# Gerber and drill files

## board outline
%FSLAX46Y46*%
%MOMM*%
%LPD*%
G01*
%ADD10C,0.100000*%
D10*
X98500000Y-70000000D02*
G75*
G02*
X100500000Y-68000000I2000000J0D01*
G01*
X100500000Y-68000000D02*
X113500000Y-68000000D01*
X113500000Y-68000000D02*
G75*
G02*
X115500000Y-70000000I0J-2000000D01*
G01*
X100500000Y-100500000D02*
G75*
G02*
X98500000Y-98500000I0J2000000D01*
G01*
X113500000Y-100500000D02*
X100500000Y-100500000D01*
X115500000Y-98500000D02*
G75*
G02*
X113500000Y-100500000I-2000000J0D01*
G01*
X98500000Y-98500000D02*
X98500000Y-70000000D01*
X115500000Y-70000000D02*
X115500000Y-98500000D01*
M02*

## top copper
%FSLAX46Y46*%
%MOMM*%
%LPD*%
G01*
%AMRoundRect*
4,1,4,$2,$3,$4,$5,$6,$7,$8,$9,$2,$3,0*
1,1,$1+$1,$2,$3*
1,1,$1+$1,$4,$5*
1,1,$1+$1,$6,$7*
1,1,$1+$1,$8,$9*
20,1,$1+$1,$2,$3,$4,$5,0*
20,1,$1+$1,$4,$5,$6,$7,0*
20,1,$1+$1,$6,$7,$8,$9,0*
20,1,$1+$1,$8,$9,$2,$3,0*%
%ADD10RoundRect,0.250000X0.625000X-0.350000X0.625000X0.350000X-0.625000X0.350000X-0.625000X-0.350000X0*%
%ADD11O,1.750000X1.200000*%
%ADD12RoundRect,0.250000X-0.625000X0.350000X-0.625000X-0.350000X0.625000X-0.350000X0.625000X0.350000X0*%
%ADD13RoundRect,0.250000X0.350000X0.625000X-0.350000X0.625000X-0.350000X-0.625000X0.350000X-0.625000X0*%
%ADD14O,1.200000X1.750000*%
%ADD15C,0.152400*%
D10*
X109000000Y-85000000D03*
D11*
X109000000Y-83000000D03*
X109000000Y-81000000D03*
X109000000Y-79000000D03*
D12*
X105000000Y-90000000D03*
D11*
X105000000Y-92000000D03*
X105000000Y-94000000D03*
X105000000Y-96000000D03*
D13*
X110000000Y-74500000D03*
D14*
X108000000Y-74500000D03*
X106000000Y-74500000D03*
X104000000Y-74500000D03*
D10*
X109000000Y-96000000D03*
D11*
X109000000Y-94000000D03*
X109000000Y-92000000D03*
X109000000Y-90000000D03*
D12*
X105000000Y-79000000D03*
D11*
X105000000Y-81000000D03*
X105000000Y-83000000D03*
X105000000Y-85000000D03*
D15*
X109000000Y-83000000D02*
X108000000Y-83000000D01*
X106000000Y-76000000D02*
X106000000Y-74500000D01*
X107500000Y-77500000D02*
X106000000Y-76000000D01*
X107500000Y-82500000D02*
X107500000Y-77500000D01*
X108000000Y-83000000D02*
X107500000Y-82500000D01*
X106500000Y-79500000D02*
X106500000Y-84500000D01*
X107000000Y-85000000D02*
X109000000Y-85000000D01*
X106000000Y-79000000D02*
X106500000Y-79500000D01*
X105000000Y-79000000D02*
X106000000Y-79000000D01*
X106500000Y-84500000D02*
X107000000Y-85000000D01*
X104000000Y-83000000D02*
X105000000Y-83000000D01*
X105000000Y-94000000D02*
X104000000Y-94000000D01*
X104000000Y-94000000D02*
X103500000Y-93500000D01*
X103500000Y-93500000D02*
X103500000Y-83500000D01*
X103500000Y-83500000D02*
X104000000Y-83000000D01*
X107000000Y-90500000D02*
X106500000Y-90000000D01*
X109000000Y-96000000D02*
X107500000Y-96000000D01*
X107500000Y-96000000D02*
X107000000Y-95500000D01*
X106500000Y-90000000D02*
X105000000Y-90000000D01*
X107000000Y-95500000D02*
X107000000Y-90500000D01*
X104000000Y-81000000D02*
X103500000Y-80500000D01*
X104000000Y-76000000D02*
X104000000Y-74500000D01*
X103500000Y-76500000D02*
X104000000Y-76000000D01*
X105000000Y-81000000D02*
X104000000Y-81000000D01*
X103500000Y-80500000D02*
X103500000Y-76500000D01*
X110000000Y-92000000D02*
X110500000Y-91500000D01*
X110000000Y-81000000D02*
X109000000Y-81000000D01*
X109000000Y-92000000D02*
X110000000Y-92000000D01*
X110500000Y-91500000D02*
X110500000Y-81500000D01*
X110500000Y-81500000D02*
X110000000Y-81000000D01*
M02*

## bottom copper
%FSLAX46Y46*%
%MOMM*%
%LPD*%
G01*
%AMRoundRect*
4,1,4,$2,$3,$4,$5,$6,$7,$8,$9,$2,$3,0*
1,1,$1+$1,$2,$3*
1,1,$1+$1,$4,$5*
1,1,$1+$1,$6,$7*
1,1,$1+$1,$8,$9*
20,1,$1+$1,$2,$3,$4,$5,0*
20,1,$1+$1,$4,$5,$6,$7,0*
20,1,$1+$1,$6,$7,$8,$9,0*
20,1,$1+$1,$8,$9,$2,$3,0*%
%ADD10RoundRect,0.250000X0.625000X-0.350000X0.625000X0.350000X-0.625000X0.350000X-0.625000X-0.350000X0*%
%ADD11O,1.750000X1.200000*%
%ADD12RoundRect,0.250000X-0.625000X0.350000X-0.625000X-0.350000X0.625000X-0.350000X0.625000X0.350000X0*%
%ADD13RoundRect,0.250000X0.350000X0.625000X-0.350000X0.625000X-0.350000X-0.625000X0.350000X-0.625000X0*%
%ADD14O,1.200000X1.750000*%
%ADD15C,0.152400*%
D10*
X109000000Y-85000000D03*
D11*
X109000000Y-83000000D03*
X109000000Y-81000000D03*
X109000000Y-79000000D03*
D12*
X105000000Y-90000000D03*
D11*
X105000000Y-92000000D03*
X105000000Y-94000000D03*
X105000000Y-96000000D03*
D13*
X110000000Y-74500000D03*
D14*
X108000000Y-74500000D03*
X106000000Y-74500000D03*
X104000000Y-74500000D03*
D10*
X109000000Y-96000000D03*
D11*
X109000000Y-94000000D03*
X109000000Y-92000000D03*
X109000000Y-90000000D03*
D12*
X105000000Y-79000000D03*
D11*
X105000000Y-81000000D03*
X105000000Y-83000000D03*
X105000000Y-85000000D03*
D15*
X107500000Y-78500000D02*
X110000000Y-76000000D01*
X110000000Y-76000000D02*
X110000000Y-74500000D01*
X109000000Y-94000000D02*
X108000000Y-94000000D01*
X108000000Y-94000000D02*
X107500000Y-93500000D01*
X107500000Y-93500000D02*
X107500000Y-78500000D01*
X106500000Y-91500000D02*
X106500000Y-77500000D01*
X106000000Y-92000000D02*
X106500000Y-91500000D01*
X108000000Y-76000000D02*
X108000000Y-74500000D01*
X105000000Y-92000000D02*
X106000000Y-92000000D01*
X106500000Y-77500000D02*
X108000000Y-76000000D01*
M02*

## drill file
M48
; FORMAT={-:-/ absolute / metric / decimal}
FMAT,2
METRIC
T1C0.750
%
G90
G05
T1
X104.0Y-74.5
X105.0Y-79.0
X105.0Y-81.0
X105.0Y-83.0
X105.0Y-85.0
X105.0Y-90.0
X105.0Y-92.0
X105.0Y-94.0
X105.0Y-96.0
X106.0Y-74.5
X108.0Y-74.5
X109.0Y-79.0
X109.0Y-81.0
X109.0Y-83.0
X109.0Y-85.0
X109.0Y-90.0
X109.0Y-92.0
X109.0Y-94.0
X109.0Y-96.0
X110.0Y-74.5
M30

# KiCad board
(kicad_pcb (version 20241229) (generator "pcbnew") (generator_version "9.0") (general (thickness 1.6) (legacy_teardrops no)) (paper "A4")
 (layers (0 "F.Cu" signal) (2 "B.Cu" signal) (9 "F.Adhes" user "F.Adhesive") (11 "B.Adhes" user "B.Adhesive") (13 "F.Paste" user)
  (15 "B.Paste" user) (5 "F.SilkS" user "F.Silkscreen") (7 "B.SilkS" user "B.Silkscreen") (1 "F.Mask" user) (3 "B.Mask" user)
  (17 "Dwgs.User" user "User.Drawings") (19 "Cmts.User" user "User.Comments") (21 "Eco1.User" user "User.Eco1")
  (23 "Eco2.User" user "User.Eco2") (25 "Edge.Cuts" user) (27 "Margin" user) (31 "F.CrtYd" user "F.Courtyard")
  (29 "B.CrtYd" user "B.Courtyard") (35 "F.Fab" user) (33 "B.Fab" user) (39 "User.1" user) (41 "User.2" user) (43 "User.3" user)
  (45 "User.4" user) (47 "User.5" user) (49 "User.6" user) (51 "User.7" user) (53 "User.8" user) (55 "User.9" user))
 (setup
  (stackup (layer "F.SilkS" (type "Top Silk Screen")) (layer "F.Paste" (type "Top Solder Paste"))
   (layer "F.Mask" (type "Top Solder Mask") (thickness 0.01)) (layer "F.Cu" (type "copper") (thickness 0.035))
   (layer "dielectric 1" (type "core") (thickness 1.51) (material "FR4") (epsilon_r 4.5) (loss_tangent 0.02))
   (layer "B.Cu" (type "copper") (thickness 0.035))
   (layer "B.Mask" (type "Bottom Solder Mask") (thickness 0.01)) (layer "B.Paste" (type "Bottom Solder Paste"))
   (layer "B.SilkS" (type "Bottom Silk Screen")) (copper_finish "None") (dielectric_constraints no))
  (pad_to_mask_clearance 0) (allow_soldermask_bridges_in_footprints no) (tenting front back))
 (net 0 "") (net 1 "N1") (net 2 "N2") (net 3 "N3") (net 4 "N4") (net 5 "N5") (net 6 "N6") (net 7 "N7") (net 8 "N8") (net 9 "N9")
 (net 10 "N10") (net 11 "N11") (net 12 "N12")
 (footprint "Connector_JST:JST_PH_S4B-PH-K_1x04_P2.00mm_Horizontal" (layer "F.Cu") (at 109 85 90)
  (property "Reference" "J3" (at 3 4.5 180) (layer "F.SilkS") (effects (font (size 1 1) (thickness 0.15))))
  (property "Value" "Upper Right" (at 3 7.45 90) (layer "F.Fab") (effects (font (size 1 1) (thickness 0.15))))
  (pad "1" thru_hole roundrect (at 0 0 90) (size 1.2 1.75) (drill 0.75) (layers "*.Cu" "*.Mask") (remove_unused_layers no)
   (roundrect_rratio 0.208333) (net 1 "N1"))
  (pad "2" thru_hole oval (at 2 0 90) (size 1.2 1.75) (drill 0.75) (layers "*.Cu" "*.Mask") (remove_unused_layers no) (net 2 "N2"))
  (pad "3" thru_hole oval (at 4 0 90) (size 1.2 1.75) (drill 0.75) (layers "*.Cu" "*.Mask") (remove_unused_layers no) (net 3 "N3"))
  (pad "4" thru_hole oval (at 6 0 90) (size 1.2 1.75) (drill 0.75) (layers "*.Cu" "*.Mask") (remove_unused_layers no) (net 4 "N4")))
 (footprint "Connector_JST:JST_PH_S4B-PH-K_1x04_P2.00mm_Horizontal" (layer "F.Cu") (at 105 90 -90)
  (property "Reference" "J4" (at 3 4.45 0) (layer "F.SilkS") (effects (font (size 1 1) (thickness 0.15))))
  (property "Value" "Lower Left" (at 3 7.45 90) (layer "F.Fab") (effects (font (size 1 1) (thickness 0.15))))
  (pad "1" thru_hole roundrect (at 0 0 270) (size 1.2 1.75) (drill 0.75) (layers "*.Cu" "*.Mask") (remove_unused_layers no)
   (roundrect_rratio 0.208333) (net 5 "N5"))
  (pad "2" thru_hole oval (at 2 0 270) (size 1.2 1.75) (drill 0.75) (layers "*.Cu" "*.Mask") (remove_unused_layers no) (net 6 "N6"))
  (pad "3" thru_hole oval (at 4 0 270) (size 1.2 1.75) (drill 0.75) (layers "*.Cu" "*.Mask") (remove_unused_layers no) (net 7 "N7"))
  (pad "4" thru_hole oval (at 6 0 270) (size 1.2 1.75) (drill 0.75) (layers "*.Cu" "*.Mask") (remove_unused_layers no) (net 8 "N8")))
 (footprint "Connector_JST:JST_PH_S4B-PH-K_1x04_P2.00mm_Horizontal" (layer "F.Cu") (at 110 74.5 180)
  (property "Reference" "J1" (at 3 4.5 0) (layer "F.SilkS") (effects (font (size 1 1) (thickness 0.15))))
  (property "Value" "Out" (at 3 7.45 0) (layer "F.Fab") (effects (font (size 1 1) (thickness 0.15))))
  (pad "1" thru_hole roundrect (at 0 0 180) (size 1.2 1.75) (drill 0.75) (layers "*.Cu" "*.Mask") (remove_unused_layers no)
   (roundrect_rratio 0.208333) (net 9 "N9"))
  (pad "2" thru_hole oval (at 2 0 180) (size 1.2 1.75) (drill 0.75) (layers "*.Cu" "*.Mask") (remove_unused_layers no) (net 6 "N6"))
  (pad "3" thru_hole oval (at 4 0 180) (size 1.2 1.75) (drill 0.75) (layers "*.Cu" "*.Mask") (remove_unused_layers no) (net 2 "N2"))
  (pad "4" thru_hole oval (at 6 0 180) (size 1.2 1.75) (drill 0.75) (layers "*.Cu" "*.Mask") (remove_unused_layers no) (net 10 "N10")))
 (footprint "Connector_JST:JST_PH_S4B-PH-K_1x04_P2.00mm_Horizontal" (layer "F.Cu") (at 109 96 90)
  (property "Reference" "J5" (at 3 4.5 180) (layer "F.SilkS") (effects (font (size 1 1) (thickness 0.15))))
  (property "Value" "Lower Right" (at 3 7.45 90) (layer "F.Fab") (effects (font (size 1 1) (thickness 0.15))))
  (pad "1" thru_hole roundrect (at 0 0 90) (size 1.2 1.75) (drill 0.75) (layers "*.Cu" "*.Mask") (remove_unused_layers no)
   (roundrect_rratio 0.208333) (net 5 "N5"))
  (pad "2" thru_hole oval (at 2 0 90) (size 1.2 1.75) (drill 0.75) (layers "*.Cu" "*.Mask") (remove_unused_layers no) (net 9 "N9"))
  (pad "3" thru_hole oval (at 4 0 90) (size 1.2 1.75) (drill 0.75) (layers "*.Cu" "*.Mask") (remove_unused_layers no) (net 3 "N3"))
  (pad "4" thru_hole oval (at 6 0 90) (size 1.2 1.75) (drill 0.75) (layers "*.Cu" "*.Mask") (remove_unused_layers no) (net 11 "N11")))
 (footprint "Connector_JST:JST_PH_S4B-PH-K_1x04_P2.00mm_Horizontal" (layer "F.Cu") (at 105 79 -90)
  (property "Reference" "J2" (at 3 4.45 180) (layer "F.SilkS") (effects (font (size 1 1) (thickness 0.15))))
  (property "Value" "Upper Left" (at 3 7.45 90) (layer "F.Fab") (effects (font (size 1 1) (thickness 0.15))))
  (pad "1" thru_hole roundrect (at 0 0 270) (size 1.2 1.75) (drill 0.75) (layers "*.Cu" "*.Mask") (remove_unused_layers no)
   (roundrect_rratio 0.208333) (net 1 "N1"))
  (pad "2" thru_hole oval (at 2 0 270) (size 1.2 1.75) (drill 0.75) (layers "*.Cu" "*.Mask") (remove_unused_layers no) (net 10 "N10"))
  (pad "3" thru_hole oval (at 4 0 270) (size 1.2 1.75) (drill 0.75) (layers "*.Cu" "*.Mask") (remove_unused_layers no) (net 7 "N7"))
  (pad "4" thru_hole oval (at 6 0 270) (size 1.2 1.75) (drill 0.75) (layers "*.Cu" "*.Mask") (remove_unused_layers no) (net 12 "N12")))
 (gr_arc (start 98.5 70) (mid 99.085786 68.585786) (end 100.5 68) (stroke (width 0.1) (type default)) (layer "Edge.Cuts"))
 (gr_line (start 100.5 68) (end 113.5 68) (stroke (width 0.1) (type default)) (layer "Edge.Cuts"))
 (gr_arc (start 113.5 68) (mid 114.914214 68.585786) (end 115.5 70) (stroke (width 0.1) (type default)) (layer "Edge.Cuts"))
 (gr_arc (start 100.5 100.5) (mid 99.085786 99.914214) (end 98.5 98.5) (stroke (width 0.1) (type default)) (layer "Edge.Cuts"))
 (gr_line (start 113.5 100.5) (end 100.5 100.5) (stroke (width 0.1) (type default)) (layer "Edge.Cuts"))
 (gr_arc (start 115.5 98.5) (mid 114.914214 99.914214) (end 113.5 100.5) (stroke (width 0.1) (type default)) (layer "Edge.Cuts"))
 (gr_line (start 98.5 98.5) (end 98.5 70) (stroke (width 0.1) (type default)) (layer "Edge.Cuts"))
 (gr_line (start 115.5 70) (end 115.5 98.5) (stroke (width 0.1) (type default)) (layer "Edge.Cuts"))
 (segment (start 107.5 78.5) (end 110 76) (width 0.1524) (layer "B.Cu") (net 9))
 (segment (start 110 76) (end 110 74.5) (width 0.1524) (layer "B.Cu") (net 9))
 (segment (start 109 94) (end 108 94) (width 0.1524) (layer "B.Cu") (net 9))
 (segment (start 108 94) (end 107.5 93.5) (width 0.1524) (layer "B.Cu") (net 9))
 (segment (start 107.5 93.5) (end 107.5 78.5) (width 0.1524) (layer "B.Cu") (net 9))
 (segment (start 106.5 91.5) (end 106.5 77.5) (width 0.1524) (layer "B.Cu") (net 6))
 (segment (start 106 92) (end 106.5 91.5) (width 0.1524) (layer "B.Cu") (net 6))
 (segment (start 108 76) (end 108 74.5) (width 0.1524) (layer "B.Cu") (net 6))
 (segment (start 105 92) (end 106 92) (width 0.1524) (layer "B.Cu") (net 6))
 (segment (start 106.5 77.5) (end 108 76) (width 0.1524) (layer "B.Cu") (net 6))
 (segment (start 109 83) (end 108 83) (width 0.1524) (layer "F.Cu") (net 2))
 (segment (start 106 76) (end 106 74.5) (width 0.1524) (layer "F.Cu") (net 2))
 (segment (start 107.5 77.5) (end 106 76) (width 0.1524) (layer "F.Cu") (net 2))
 (segment (start 107.5 82.5) (end 107.5 77.5) (width 0.1524) (layer "F.Cu") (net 2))
 (segment (start 108 83) (end 107.5 82.5) (width 0.1524) (layer "F.Cu") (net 2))
 (segment (start 106.5 79.5) (end 106.5 84.5) (width 0.1524) (layer "F.Cu") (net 1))
 (segment (start 107 85) (end 109 85) (width 0.1524) (layer "F.Cu") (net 1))
 (segment (start 106 79) (end 106.5 79.5) (width 0.1524) (layer "F.Cu") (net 1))
 (segment (start 105 79) (end 106 79) (width 0.1524) (layer "F.Cu") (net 1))
 (segment (start 106.5 84.5) (end 107 85) (width 0.1524) (layer "F.Cu") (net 1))
 (segment (start 104 83) (end 105 83) (width 0.1524) (layer "F.Cu") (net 7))
 (segment (start 105 94) (end 104 94) (width 0.1524) (layer "F.Cu") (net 7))
 (segment (start 104 94) (end 103.5 93.5) (width 0.1524) (layer "F.Cu") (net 7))
 (segment (start 103.5 93.5) (end 103.5 83.5) (width 0.1524) (layer "F.Cu") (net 7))
 (segment (start 103.5 83.5) (end 104 83) (width 0.1524) (layer "F.Cu") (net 7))
 (segment (start 107 90.5) (end 106.5 90) (width 0.1524) (layer "F.Cu") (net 5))
 (segment (start 109 96) (end 107.5 96) (width 0.1524) (layer "F.Cu") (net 5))
 (segment (start 107.5 96) (end 107 95.5) (width 0.1524) (layer "F.Cu") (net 5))
 (segment (start 106.5 90) (end 105 90) (width 0.1524) (layer "F.Cu") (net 5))
 (segment (start 107 95.5) (end 107 90.5) (width 0.1524) (layer "F.Cu") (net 5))
 (segment (start 104 81) (end 103.5 80.5) (width 0.1524) (layer "F.Cu") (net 10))
 (segment (start 104 76) (end 104 74.5) (width 0.1524) (layer "F.Cu") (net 10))
 (segment (start 103.5 76.5) (end 104 76) (width 0.1524) (layer "F.Cu") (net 10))
 (segment (start 105 81) (end 104 81) (width 0.1524) (layer "F.Cu") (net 10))
 (segment (start 103.5 80.5) (end 103.5 76.5) (width 0.1524) (layer "F.Cu") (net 10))
 (segment (start 110 92) (end 110.5 91.5) (width 0.1524) (layer "F.Cu") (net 3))
 (segment (start 110 81) (end 109 81) (width 0.1524) (layer "F.Cu") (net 3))
 (segment (start 109 92) (end 110 92) (width 0.1524) (layer "F.Cu") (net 3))
 (segment (start 110.5 91.5) (end 110.5 81.5) (width 0.1524) (layer "F.Cu") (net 3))
 (segment (start 110.5 81.5) (end 110 81) (width 0.1524) (layer "F.Cu") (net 3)))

